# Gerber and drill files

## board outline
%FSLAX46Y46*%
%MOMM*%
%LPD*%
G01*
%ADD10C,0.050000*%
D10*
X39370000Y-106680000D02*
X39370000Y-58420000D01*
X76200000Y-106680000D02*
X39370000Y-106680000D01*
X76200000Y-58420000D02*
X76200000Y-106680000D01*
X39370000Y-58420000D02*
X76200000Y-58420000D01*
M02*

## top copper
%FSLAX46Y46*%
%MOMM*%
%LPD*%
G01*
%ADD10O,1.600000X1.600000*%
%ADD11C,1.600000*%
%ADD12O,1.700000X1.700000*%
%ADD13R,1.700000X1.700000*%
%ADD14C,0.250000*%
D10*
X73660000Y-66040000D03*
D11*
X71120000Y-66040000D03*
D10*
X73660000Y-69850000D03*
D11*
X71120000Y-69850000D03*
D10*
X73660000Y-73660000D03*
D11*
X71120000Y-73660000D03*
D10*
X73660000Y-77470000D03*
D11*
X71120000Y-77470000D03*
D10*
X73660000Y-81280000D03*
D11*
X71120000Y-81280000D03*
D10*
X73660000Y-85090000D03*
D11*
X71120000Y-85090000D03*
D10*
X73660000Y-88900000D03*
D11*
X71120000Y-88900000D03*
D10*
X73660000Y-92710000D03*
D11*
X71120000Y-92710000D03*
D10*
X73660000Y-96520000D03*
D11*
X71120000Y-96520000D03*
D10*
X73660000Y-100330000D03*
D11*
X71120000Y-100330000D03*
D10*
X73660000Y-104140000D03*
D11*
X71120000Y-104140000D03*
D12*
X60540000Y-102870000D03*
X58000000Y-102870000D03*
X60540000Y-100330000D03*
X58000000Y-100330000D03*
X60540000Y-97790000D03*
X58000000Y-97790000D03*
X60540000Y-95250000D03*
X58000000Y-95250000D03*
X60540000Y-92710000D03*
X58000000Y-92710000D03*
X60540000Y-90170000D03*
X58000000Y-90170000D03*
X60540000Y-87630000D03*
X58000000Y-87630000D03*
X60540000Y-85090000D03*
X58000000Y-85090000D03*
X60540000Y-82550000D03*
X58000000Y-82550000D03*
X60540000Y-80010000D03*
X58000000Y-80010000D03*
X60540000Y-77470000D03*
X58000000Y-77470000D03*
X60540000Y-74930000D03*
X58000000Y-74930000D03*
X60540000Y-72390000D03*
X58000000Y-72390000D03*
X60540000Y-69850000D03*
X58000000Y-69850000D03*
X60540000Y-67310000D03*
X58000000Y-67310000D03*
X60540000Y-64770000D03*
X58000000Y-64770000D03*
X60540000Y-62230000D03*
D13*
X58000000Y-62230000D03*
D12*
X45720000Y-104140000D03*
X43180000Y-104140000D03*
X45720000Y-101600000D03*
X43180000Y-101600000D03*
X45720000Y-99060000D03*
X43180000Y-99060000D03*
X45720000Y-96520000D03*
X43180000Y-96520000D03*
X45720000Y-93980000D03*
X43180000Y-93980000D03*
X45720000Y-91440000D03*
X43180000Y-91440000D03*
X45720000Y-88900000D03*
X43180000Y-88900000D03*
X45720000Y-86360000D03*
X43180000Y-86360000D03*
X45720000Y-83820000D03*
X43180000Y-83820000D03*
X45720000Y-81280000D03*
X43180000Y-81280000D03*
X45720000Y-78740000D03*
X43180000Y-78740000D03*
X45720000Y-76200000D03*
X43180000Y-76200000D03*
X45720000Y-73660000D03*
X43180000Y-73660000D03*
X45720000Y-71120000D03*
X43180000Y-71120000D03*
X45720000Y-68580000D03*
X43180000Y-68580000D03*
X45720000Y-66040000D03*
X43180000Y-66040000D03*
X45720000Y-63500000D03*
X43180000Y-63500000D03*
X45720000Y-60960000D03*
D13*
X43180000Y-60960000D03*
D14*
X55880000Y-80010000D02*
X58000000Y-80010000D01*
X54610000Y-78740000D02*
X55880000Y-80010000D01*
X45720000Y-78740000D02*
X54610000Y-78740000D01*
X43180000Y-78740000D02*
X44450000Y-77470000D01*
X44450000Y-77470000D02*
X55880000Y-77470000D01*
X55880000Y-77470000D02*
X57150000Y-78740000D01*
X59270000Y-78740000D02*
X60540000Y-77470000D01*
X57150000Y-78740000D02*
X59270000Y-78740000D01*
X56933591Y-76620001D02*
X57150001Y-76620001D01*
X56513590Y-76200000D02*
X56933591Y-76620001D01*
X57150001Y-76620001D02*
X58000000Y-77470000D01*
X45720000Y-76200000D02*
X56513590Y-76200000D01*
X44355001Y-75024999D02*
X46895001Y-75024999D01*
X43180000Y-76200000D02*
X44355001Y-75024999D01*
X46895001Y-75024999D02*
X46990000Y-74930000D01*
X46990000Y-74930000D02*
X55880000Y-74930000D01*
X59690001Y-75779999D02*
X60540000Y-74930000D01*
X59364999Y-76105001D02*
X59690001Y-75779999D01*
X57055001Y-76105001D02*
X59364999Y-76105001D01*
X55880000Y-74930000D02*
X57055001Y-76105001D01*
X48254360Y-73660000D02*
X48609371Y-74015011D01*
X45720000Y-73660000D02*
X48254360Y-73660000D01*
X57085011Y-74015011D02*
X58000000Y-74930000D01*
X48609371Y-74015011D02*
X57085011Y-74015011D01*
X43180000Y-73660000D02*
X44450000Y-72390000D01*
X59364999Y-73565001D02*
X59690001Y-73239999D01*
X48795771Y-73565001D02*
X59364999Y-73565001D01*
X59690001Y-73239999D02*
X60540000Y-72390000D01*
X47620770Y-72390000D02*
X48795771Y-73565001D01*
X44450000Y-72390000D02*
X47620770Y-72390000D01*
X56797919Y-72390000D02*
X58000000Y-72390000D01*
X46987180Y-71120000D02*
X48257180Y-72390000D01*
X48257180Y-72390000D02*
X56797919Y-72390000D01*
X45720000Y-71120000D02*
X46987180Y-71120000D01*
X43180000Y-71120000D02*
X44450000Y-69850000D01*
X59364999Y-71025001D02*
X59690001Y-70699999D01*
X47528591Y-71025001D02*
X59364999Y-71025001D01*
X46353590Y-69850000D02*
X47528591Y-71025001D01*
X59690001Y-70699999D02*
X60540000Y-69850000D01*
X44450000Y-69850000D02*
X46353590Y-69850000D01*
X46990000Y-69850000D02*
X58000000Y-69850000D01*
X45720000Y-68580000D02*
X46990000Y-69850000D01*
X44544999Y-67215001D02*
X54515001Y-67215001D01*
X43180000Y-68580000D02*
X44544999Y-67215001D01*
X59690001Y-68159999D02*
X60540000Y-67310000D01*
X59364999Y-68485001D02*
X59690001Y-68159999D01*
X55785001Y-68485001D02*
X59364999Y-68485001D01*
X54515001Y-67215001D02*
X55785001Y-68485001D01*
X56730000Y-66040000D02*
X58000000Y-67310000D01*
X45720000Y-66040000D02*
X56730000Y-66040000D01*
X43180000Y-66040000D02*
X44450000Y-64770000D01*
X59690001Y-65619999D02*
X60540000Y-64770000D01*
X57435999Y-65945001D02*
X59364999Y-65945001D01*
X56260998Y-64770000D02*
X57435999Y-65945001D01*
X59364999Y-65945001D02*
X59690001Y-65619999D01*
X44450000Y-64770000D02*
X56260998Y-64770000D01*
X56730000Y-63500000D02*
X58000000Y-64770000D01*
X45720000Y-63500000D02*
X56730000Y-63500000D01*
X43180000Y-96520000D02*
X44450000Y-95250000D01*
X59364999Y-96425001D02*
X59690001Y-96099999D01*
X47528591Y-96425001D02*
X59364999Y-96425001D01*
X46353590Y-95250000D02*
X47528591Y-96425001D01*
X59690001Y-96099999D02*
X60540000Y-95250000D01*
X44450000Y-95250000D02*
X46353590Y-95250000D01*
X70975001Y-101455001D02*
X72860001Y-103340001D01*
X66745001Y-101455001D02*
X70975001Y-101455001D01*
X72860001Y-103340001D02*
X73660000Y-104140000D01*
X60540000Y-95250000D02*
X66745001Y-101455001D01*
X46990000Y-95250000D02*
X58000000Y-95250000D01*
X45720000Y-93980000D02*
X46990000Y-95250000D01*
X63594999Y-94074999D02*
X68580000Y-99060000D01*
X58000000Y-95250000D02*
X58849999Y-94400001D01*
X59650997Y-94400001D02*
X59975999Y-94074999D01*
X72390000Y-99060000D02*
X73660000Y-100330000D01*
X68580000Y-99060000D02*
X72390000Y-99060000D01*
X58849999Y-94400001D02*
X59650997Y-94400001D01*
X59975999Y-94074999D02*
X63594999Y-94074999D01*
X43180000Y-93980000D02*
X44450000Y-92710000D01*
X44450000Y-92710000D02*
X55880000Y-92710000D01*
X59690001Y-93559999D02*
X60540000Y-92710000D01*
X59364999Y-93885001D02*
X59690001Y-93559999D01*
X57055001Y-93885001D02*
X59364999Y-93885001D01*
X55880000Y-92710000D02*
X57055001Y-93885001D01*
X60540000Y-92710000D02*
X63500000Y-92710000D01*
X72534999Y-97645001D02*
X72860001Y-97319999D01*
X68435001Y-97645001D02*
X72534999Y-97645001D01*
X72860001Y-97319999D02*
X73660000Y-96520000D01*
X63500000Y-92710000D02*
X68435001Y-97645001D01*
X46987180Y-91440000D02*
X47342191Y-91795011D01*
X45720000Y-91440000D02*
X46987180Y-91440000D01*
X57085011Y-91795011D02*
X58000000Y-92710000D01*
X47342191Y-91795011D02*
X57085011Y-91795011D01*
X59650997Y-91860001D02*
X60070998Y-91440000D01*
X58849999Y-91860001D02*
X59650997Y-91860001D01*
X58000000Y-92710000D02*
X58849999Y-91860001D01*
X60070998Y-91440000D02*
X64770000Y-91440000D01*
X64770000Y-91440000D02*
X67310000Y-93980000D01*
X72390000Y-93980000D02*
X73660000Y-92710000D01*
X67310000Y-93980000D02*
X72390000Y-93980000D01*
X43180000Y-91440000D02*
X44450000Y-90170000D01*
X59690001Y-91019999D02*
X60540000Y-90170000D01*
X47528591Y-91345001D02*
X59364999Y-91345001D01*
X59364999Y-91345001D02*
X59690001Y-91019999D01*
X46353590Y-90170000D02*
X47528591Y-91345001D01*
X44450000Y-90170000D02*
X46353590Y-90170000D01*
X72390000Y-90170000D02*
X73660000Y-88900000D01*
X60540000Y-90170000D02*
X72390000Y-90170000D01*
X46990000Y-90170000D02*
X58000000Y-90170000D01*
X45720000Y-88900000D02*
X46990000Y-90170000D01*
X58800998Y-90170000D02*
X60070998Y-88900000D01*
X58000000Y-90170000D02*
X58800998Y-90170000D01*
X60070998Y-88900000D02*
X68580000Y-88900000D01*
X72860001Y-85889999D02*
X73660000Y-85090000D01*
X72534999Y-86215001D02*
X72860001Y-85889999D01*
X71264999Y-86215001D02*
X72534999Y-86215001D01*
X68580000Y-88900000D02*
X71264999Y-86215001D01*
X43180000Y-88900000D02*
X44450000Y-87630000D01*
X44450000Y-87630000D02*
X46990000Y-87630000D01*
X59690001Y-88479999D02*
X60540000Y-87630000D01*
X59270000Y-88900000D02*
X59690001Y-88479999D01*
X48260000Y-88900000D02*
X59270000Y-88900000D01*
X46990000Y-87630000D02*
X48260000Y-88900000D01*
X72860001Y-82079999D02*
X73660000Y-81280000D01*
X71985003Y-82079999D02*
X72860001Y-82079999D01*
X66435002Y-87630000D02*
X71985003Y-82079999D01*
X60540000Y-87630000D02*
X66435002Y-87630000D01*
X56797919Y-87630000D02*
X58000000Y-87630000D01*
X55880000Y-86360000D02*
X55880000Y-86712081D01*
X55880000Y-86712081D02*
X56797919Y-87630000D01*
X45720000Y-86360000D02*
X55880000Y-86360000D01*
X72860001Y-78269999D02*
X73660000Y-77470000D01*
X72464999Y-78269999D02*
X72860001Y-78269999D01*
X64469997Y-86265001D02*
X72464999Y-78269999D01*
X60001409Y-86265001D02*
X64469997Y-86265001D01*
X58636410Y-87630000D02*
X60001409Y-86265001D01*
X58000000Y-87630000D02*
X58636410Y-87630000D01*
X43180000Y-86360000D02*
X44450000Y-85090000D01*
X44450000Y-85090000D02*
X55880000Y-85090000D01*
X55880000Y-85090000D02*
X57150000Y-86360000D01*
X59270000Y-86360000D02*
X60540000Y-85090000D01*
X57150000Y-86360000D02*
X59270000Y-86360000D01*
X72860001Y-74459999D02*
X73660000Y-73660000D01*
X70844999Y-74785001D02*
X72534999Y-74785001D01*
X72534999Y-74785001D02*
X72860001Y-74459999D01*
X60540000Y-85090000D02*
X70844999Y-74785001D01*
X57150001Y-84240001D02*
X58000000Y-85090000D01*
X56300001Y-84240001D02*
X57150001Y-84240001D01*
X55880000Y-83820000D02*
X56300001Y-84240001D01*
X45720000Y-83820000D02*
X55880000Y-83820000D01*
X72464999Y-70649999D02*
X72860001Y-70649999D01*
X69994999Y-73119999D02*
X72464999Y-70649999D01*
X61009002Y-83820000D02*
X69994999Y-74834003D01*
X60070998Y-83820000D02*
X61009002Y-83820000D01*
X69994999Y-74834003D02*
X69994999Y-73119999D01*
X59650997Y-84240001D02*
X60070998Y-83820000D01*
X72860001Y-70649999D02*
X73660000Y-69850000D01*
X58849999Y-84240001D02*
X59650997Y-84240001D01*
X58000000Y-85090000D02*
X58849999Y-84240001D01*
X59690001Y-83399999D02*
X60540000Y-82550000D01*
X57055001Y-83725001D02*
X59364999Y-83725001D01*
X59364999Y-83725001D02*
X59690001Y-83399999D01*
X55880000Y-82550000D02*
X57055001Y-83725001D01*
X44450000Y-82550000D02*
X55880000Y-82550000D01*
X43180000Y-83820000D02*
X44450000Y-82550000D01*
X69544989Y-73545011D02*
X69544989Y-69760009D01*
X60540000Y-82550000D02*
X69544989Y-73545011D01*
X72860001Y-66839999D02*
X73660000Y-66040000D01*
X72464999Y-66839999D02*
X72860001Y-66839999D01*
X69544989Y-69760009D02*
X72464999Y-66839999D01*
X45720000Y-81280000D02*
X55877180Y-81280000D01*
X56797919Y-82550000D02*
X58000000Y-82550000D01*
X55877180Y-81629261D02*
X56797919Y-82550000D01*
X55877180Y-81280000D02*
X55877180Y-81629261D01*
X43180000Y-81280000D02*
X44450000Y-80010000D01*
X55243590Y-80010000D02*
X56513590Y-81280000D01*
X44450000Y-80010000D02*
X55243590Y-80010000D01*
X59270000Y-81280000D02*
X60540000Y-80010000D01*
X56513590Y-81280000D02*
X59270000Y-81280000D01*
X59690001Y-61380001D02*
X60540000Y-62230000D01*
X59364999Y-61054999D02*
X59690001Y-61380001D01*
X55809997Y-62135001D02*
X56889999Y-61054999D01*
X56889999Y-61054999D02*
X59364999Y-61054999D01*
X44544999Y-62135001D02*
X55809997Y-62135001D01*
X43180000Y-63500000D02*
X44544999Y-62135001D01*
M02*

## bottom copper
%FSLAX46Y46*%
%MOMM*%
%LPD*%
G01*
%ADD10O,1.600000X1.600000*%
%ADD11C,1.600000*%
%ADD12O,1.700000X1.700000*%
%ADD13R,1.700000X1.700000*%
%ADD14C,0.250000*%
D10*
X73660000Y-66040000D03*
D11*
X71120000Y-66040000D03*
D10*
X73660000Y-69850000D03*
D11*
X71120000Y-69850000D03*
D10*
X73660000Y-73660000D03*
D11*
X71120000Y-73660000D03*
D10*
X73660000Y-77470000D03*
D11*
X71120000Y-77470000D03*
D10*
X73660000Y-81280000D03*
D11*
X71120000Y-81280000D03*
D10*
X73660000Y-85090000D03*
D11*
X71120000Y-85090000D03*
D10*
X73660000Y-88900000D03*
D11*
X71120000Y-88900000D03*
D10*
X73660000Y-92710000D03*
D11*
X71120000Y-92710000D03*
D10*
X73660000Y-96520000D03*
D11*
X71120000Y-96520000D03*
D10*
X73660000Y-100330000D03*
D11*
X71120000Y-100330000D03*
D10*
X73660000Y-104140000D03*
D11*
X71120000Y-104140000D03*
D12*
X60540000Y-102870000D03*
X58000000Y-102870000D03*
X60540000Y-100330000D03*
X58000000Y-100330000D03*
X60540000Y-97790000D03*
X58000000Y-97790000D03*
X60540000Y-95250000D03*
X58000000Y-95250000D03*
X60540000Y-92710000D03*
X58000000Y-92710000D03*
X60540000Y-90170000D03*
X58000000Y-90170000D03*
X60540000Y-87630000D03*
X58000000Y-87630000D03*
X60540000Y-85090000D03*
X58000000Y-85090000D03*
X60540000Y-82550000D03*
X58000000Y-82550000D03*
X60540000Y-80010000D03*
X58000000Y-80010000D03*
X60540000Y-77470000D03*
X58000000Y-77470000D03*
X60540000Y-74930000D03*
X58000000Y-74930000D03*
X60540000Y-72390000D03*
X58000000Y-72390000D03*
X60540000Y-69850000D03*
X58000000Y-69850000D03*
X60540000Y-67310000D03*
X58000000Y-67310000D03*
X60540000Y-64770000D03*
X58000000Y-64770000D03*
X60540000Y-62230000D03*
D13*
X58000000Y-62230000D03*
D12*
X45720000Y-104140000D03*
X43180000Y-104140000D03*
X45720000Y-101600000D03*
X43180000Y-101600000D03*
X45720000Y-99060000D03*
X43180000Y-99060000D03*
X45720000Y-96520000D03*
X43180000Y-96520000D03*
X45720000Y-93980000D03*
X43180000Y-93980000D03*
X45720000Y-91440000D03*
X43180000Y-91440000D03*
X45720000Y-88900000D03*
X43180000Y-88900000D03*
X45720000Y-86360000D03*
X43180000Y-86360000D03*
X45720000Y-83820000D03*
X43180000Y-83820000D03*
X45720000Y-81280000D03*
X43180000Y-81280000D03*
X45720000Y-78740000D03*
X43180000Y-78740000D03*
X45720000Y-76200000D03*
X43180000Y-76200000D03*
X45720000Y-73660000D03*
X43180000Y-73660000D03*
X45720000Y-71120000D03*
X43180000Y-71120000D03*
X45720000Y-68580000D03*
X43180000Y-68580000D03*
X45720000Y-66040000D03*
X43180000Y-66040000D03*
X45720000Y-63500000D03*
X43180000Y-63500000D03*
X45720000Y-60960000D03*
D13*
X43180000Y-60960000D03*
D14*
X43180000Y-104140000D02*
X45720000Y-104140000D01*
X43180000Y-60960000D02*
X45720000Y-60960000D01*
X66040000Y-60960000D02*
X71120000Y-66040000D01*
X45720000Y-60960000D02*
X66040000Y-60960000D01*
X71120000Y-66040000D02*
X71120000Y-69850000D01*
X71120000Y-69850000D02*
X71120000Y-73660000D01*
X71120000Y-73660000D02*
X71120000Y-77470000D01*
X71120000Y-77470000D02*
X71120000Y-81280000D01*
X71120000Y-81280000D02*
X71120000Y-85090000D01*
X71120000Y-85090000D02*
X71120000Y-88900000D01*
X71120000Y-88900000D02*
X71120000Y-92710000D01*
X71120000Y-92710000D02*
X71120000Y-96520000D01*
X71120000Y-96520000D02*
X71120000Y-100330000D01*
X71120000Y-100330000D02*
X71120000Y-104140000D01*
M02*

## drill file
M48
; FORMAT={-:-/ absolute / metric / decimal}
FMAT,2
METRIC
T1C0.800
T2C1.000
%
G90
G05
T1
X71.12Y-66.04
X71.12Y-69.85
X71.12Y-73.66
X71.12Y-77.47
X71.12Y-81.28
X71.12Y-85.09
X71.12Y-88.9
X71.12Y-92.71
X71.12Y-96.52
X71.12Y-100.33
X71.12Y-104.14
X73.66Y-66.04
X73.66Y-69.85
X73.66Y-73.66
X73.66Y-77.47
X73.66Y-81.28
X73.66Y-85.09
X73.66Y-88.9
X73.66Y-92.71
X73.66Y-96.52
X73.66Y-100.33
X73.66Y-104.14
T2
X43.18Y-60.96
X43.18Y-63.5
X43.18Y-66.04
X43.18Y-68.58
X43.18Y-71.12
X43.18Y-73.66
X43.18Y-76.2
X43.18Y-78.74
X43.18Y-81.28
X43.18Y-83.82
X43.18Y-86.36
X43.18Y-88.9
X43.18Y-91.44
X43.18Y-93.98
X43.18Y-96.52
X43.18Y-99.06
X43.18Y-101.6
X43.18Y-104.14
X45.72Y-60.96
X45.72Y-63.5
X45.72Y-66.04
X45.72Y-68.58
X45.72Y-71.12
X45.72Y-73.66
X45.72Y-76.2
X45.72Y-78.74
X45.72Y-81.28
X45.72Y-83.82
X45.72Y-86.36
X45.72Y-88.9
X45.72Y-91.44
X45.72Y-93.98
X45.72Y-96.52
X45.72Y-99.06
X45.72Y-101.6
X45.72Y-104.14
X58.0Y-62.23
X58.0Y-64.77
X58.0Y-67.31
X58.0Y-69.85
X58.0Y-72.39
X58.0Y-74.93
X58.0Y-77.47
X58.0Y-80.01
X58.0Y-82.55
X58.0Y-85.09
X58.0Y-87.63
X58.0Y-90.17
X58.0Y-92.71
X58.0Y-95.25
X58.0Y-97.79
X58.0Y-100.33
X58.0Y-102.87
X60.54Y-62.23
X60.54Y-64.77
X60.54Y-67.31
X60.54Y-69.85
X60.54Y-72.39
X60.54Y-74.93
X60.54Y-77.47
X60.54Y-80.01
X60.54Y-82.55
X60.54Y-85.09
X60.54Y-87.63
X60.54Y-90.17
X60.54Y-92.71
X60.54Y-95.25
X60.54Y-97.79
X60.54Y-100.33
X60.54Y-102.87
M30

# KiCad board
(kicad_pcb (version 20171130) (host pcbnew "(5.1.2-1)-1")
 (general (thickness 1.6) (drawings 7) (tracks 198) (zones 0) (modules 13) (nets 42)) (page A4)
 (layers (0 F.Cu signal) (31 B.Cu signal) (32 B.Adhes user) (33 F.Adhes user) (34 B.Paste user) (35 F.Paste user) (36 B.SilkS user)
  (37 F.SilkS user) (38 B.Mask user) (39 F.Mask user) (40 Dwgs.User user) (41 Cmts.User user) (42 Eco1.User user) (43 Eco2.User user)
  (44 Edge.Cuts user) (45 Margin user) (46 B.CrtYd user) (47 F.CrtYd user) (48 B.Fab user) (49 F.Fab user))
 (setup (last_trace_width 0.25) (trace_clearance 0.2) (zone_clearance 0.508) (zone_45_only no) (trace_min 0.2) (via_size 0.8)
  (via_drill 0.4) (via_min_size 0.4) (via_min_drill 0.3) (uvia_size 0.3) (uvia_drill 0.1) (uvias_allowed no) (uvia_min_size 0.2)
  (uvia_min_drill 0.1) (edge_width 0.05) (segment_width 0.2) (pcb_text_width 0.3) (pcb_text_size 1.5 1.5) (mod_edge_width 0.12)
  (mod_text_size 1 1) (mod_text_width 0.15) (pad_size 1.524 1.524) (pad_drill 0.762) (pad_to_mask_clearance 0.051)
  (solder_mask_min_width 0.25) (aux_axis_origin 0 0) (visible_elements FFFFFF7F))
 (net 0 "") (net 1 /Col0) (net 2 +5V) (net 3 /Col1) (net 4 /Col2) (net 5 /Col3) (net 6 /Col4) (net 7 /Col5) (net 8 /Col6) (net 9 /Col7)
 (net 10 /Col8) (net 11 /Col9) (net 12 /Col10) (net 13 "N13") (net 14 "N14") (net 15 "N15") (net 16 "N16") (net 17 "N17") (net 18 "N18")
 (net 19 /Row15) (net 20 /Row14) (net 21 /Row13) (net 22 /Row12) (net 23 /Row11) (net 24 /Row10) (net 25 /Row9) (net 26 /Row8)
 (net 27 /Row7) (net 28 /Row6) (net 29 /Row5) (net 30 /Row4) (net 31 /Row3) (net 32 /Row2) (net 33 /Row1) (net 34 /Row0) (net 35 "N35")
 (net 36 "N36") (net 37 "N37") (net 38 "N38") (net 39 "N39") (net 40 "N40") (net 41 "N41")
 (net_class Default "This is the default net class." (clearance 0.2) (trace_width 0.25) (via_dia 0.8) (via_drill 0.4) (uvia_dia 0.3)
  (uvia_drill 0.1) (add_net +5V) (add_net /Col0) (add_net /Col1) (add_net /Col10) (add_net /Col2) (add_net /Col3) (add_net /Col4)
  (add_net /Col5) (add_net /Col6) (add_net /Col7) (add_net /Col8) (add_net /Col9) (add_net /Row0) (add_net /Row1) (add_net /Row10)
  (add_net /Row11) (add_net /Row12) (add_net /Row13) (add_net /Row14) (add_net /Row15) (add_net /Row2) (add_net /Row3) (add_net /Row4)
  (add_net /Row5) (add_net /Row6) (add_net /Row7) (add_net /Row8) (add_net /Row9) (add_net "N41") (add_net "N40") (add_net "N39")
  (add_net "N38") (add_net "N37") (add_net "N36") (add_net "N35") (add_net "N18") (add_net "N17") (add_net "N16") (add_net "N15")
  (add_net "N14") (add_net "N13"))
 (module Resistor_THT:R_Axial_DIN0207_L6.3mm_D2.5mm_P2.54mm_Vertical (layer F.Cu) (at 71.12 66.04)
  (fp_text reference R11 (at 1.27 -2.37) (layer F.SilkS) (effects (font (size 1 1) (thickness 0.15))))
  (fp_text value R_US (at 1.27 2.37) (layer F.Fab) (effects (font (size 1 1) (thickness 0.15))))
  (pad 2 thru_hole oval (at 2.54 0) (size 1.6 1.6) (drill 0.8) (layers *.Cu *.Mask) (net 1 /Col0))
  (pad 1 thru_hole circle (at 0 0) (size 1.6 1.6) (drill 0.8) (layers *.Cu *.Mask) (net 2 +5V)))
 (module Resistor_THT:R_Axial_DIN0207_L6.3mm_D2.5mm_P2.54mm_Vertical (layer F.Cu) (at 71.12 69.85)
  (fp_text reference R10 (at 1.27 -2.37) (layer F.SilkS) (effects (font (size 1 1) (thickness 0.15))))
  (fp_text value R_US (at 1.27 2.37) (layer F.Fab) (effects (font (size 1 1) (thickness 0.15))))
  (pad 2 thru_hole oval (at 2.54 0) (size 1.6 1.6) (drill 0.8) (layers *.Cu *.Mask) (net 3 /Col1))
  (pad 1 thru_hole circle (at 0 0) (size 1.6 1.6) (drill 0.8) (layers *.Cu *.Mask) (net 2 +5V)))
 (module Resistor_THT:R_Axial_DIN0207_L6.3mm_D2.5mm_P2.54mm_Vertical (layer F.Cu) (at 71.12 73.66)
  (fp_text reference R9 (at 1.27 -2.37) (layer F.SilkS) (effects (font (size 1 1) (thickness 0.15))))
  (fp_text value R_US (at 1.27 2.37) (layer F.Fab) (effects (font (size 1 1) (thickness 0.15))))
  (pad 2 thru_hole oval (at 2.54 0) (size 1.6 1.6) (drill 0.8) (layers *.Cu *.Mask) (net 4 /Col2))
  (pad 1 thru_hole circle (at 0 0) (size 1.6 1.6) (drill 0.8) (layers *.Cu *.Mask) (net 2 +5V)))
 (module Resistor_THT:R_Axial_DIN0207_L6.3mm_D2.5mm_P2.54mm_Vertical (layer F.Cu) (at 71.12 77.47)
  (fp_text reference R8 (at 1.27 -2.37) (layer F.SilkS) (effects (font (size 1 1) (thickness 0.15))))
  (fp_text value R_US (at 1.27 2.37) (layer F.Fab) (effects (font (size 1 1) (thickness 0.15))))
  (pad 2 thru_hole oval (at 2.54 0) (size 1.6 1.6) (drill 0.8) (layers *.Cu *.Mask) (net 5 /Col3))
  (pad 1 thru_hole circle (at 0 0) (size 1.6 1.6) (drill 0.8) (layers *.Cu *.Mask) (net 2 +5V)))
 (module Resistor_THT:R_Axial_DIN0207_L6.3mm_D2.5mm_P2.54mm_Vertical (layer F.Cu) (at 71.12 81.28)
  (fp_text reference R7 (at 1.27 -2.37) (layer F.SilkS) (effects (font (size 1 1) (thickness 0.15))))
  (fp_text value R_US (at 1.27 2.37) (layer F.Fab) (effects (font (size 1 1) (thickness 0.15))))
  (pad 2 thru_hole oval (at 2.54 0) (size 1.6 1.6) (drill 0.8) (layers *.Cu *.Mask) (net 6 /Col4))
  (pad 1 thru_hole circle (at 0 0) (size 1.6 1.6) (drill 0.8) (layers *.Cu *.Mask) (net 2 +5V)))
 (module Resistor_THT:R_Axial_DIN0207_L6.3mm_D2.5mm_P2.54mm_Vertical (layer F.Cu) (at 71.12 85.09)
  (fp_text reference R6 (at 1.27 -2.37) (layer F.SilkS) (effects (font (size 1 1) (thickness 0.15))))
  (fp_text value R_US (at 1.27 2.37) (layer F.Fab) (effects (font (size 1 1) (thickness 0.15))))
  (pad 2 thru_hole oval (at 2.54 0) (size 1.6 1.6) (drill 0.8) (layers *.Cu *.Mask) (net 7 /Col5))
  (pad 1 thru_hole circle (at 0 0) (size 1.6 1.6) (drill 0.8) (layers *.Cu *.Mask) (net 2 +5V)))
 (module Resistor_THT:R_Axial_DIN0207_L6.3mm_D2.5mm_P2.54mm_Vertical (layer F.Cu) (at 71.12 88.9)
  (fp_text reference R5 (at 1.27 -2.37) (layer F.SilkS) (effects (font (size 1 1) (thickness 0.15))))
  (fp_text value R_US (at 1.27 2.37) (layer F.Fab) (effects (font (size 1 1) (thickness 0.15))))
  (pad 2 thru_hole oval (at 2.54 0) (size 1.6 1.6) (drill 0.8) (layers *.Cu *.Mask) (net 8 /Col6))
  (pad 1 thru_hole circle (at 0 0) (size 1.6 1.6) (drill 0.8) (layers *.Cu *.Mask) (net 2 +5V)))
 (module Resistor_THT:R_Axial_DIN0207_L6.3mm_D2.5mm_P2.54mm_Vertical (layer F.Cu) (at 71.12 92.71)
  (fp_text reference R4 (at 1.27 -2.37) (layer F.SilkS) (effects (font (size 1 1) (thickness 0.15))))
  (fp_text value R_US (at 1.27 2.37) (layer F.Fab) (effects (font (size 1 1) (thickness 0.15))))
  (pad 2 thru_hole oval (at 2.54 0) (size 1.6 1.6) (drill 0.8) (layers *.Cu *.Mask) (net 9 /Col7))
  (pad 1 thru_hole circle (at 0 0) (size 1.6 1.6) (drill 0.8) (layers *.Cu *.Mask) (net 2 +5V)))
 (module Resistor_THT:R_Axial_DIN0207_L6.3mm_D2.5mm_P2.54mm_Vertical (layer F.Cu) (at 71.12 96.52)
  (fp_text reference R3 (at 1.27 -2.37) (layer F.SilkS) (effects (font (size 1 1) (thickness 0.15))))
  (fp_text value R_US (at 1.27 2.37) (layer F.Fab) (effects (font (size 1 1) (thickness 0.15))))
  (pad 2 thru_hole oval (at 2.54 0) (size 1.6 1.6) (drill 0.8) (layers *.Cu *.Mask) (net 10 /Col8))
  (pad 1 thru_hole circle (at 0 0) (size 1.6 1.6) (drill 0.8) (layers *.Cu *.Mask) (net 2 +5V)))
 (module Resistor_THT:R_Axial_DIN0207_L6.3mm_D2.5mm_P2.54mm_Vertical (layer F.Cu) (at 71.12 100.33)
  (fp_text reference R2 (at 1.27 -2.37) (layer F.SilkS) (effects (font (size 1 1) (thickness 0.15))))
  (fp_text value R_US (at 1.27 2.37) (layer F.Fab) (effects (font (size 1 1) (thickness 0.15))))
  (pad 2 thru_hole oval (at 2.54 0) (size 1.6 1.6) (drill 0.8) (layers *.Cu *.Mask) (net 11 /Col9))
  (pad 1 thru_hole circle (at 0 0) (size 1.6 1.6) (drill 0.8) (layers *.Cu *.Mask) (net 2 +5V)))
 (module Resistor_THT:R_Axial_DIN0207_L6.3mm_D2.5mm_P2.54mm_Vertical (layer F.Cu) (at 71.12 104.14)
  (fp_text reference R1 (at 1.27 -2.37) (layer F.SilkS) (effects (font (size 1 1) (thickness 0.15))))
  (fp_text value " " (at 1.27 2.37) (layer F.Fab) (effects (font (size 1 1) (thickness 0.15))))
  (pad 2 thru_hole oval (at 2.54 0) (size 1.6 1.6) (drill 0.8) (layers *.Cu *.Mask) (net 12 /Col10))
  (pad 1 thru_hole circle (at 0 0) (size 1.6 1.6) (drill 0.8) (layers *.Cu *.Mask) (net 2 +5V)))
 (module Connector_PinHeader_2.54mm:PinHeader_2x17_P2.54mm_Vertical (layer F.Cu) (at 58 62.23)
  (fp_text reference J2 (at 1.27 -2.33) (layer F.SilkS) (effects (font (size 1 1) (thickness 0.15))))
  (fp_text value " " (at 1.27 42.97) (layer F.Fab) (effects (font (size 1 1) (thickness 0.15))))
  (pad 34 thru_hole oval (at 2.54 40.64) (size 1.7 1.7) (drill 1) (layers *.Cu *.Mask) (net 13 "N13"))
  (pad 33 thru_hole oval (at 0 40.64) (size 1.7 1.7) (drill 1) (layers *.Cu *.Mask) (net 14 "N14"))
  (pad 32 thru_hole oval (at 2.54 38.1) (size 1.7 1.7) (drill 1) (layers *.Cu *.Mask) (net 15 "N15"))
  (pad 31 thru_hole oval (at 0 38.1) (size 1.7 1.7) (drill 1) (layers *.Cu *.Mask) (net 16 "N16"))
  (pad 30 thru_hole oval (at 2.54 35.56) (size 1.7 1.7) (drill 1) (layers *.Cu *.Mask) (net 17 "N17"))
  (pad 29 thru_hole oval (at 0 35.56) (size 1.7 1.7) (drill 1) (layers *.Cu *.Mask) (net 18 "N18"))
  (pad 28 thru_hole oval (at 2.54 33.02) (size 1.7 1.7) (drill 1) (layers *.Cu *.Mask) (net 12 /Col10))
  (pad 27 thru_hole oval (at 0 33.02) (size 1.7 1.7) (drill 1) (layers *.Cu *.Mask) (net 11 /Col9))
  (pad 26 thru_hole oval (at 2.54 30.48) (size 1.7 1.7) (drill 1) (layers *.Cu *.Mask) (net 10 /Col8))
  (pad 25 thru_hole oval (at 0 30.48) (size 1.7 1.7) (drill 1) (layers *.Cu *.Mask) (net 9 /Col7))
  (pad 24 thru_hole oval (at 2.54 27.94) (size 1.7 1.7) (drill 1) (layers *.Cu *.Mask) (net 8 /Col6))
  (pad 23 thru_hole oval (at 0 27.94) (size 1.7 1.7) (drill 1) (layers *.Cu *.Mask) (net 7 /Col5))
  (pad 22 thru_hole oval (at 2.54 25.4) (size 1.7 1.7) (drill 1) (layers *.Cu *.Mask) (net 6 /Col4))
  (pad 21 thru_hole oval (at 0 25.4) (size 1.7 1.7) (drill 1) (layers *.Cu *.Mask) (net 5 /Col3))
  (pad 20 thru_hole oval (at 2.54 22.86) (size 1.7 1.7) (drill 1) (layers *.Cu *.Mask) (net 4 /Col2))
  (pad 19 thru_hole oval (at 0 22.86) (size 1.7 1.7) (drill 1) (layers *.Cu *.Mask) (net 3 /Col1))
  (pad 18 thru_hole oval (at 2.54 20.32) (size 1.7 1.7) (drill 1) (layers *.Cu *.Mask) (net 1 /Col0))
  (pad 17 thru_hole oval (at 0 20.32) (size 1.7 1.7) (drill 1) (layers *.Cu *.Mask) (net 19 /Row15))
  (pad 16 thru_hole oval (at 2.54 17.78) (size 1.7 1.7) (drill 1) (layers *.Cu *.Mask) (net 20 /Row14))
  (pad 15 thru_hole oval (at 0 17.78) (size 1.7 1.7) (drill 1) (layers *.Cu *.Mask) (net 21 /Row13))
  (pad 14 thru_hole oval (at 2.54 15.24) (size 1.7 1.7) (drill 1) (layers *.Cu *.Mask) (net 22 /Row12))
  (pad 13 thru_hole oval (at 0 15.24) (size 1.7 1.7) (drill 1) (layers *.Cu *.Mask) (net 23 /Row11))
  (pad 12 thru_hole oval (at 2.54 12.7) (size 1.7 1.7) (drill 1) (layers *.Cu *.Mask) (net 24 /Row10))
  (pad 11 thru_hole oval (at 0 12.7) (size 1.7 1.7) (drill 1) (layers *.Cu *.Mask) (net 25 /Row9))
  (pad 10 thru_hole oval (at 2.54 10.16) (size 1.7 1.7) (drill 1) (layers *.Cu *.Mask) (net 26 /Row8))
  (pad 9 thru_hole oval (at 0 10.16) (size 1.7 1.7) (drill 1) (layers *.Cu *.Mask) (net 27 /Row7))
  (pad 8 thru_hole oval (at 2.54 7.62) (size 1.7 1.7) (drill 1) (layers *.Cu *.Mask) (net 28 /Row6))
  (pad 7 thru_hole oval (at 0 7.62) (size 1.7 1.7) (drill 1) (layers *.Cu *.Mask) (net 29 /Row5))
  (pad 6 thru_hole oval (at 2.54 5.08) (size 1.7 1.7) (drill 1) (layers *.Cu *.Mask) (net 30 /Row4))
  (pad 5 thru_hole oval (at 0 5.08) (size 1.7 1.7) (drill 1) (layers *.Cu *.Mask) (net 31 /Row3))
  (pad 4 thru_hole oval (at 2.54 2.54) (size 1.7 1.7) (drill 1) (layers *.Cu *.Mask) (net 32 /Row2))
  (pad 3 thru_hole oval (at 0 2.54) (size 1.7 1.7) (drill 1) (layers *.Cu *.Mask) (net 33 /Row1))
  (pad 2 thru_hole oval (at 2.54 0) (size 1.7 1.7) (drill 1) (layers *.Cu *.Mask) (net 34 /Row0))
  (pad 1 thru_hole rect (at 0 0) (size 1.7 1.7) (drill 1) (layers *.Cu *.Mask) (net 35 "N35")))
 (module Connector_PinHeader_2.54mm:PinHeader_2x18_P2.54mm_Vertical (layer F.Cu) (at 43.18 60.96)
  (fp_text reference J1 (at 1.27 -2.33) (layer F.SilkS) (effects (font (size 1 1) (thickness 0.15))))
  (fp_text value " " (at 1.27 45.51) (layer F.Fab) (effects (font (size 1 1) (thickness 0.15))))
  (pad 36 thru_hole oval (at 2.54 43.18) (size 1.7 1.7) (drill 1) (layers *.Cu *.Mask) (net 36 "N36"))
  (pad 35 thru_hole oval (at 0 43.18) (size 1.7 1.7) (drill 1) (layers *.Cu *.Mask) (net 36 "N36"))
  (pad 34 thru_hole oval (at 2.54 40.64) (size 1.7 1.7) (drill 1) (layers *.Cu *.Mask) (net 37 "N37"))
  (pad 33 thru_hole oval (at 0 40.64) (size 1.7 1.7) (drill 1) (layers *.Cu *.Mask) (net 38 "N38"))
  (pad 32 thru_hole oval (at 2.54 38.1) (size 1.7 1.7) (drill 1) (layers *.Cu *.Mask) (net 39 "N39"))
  (pad 31 thru_hole oval (at 0 38.1) (size 1.7 1.7) (drill 1) (layers *.Cu *.Mask) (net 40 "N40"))
  (pad 30 thru_hole oval (at 2.54 35.56) (size 1.7 1.7) (drill 1) (layers *.Cu *.Mask) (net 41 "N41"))
  (pad 29 thru_hole oval (at 0 35.56) (size 1.7 1.7) (drill 1) (layers *.Cu *.Mask) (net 12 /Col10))
  (pad 28 thru_hole oval (at 2.54 33.02) (size 1.7 1.7) (drill 1) (layers *.Cu *.Mask) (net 11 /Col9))
  (pad 27 thru_hole oval (at 0 33.02) (size 1.7 1.7) (drill 1) (layers *.Cu *.Mask) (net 10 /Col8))
  (pad 26 thru_hole oval (at 2.54 30.48) (size 1.7 1.7) (drill 1) (layers *.Cu *.Mask) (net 9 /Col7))
  (pad 25 thru_hole oval (at 0 30.48) (size 1.7 1.7) (drill 1) (layers *.Cu *.Mask) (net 8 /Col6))
  (pad 24 thru_hole oval (at 2.54 27.94) (size 1.7 1.7) (drill 1) (layers *.Cu *.Mask) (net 7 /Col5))
  (pad 23 thru_hole oval (at 0 27.94) (size 1.7 1.7) (drill 1) (layers *.Cu *.Mask) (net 6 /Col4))
  (pad 22 thru_hole oval (at 2.54 25.4) (size 1.7 1.7) (drill 1) (layers *.Cu *.Mask) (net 5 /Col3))
  (pad 21 thru_hole oval (at 0 25.4) (size 1.7 1.7) (drill 1) (layers *.Cu *.Mask) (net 4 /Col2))
  (pad 20 thru_hole oval (at 2.54 22.86) (size 1.7 1.7) (drill 1) (layers *.Cu *.Mask) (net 3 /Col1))
  (pad 19 thru_hole oval (at 0 22.86) (size 1.7 1.7) (drill 1) (layers *.Cu *.Mask) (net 1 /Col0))
  (pad 18 thru_hole oval (at 2.54 20.32) (size 1.7 1.7) (drill 1) (layers *.Cu *.Mask) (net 19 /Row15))
  (pad 17 thru_hole oval (at 0 20.32) (size 1.7 1.7) (drill 1) (layers *.Cu *.Mask) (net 20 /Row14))
  (pad 16 thru_hole oval (at 2.54 17.78) (size 1.7 1.7) (drill 1) (layers *.Cu *.Mask) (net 21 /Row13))
  (pad 15 thru_hole oval (at 0 17.78) (size 1.7 1.7) (drill 1) (layers *.Cu *.Mask) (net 22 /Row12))
  (pad 14 thru_hole oval (at 2.54 15.24) (size 1.7 1.7) (drill 1) (layers *.Cu *.Mask) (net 23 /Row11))
  (pad 13 thru_hole oval (at 0 15.24) (size 1.7 1.7) (drill 1) (layers *.Cu *.Mask) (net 24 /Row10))
  (pad 12 thru_hole oval (at 2.54 12.7) (size 1.7 1.7) (drill 1) (layers *.Cu *.Mask) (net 25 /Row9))
  (pad 11 thru_hole oval (at 0 12.7) (size 1.7 1.7) (drill 1) (layers *.Cu *.Mask) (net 26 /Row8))
  (pad 10 thru_hole oval (at 2.54 10.16) (size 1.7 1.7) (drill 1) (layers *.Cu *.Mask) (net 27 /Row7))
  (pad 9 thru_hole oval (at 0 10.16) (size 1.7 1.7) (drill 1) (layers *.Cu *.Mask) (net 28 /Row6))
  (pad 8 thru_hole oval (at 2.54 7.62) (size 1.7 1.7) (drill 1) (layers *.Cu *.Mask) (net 29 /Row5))
  (pad 7 thru_hole oval (at 0 7.62) (size 1.7 1.7) (drill 1) (layers *.Cu *.Mask) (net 30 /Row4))
  (pad 6 thru_hole oval (at 2.54 5.08) (size 1.7 1.7) (drill 1) (layers *.Cu *.Mask) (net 31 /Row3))
  (pad 5 thru_hole oval (at 0 5.08) (size 1.7 1.7) (drill 1) (layers *.Cu *.Mask) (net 32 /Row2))
  (pad 4 thru_hole oval (at 2.54 2.54) (size 1.7 1.7) (drill 1) (layers *.Cu *.Mask) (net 33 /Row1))
  (pad 3 thru_hole oval (at 0 2.54) (size 1.7 1.7) (drill 1) (layers *.Cu *.Mask) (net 34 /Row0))
  (pad 2 thru_hole oval (at 2.54 0) (size 1.7 1.7) (drill 1) (layers *.Cu *.Mask) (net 2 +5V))
  (pad 1 thru_hole rect (at 0 0) (size 1.7 1.7) (drill 1) (layers *.Cu *.Mask) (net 2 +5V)))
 (gr_line (start 39.37 106.68) (end 39.37 58.42) (layer Edge.Cuts) (width 0.05))
 (gr_line (start 76.2 106.68) (end 39.37 106.68) (layer Edge.Cuts) (width 0.05))
 (gr_line (start 76.2 58.42) (end 76.2 106.68) (layer Edge.Cuts) (width 0.05))
 (gr_line (start 39.37 58.42) (end 76.2 58.42) (layer Edge.Cuts) (width 0.05))
 (segment (start 43.18 104.14) (end 45.72 104.14) (width 0.25) (layer B.Cu) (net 36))
 (segment (start 55.88 80.01) (end 58 80.01) (width 0.25) (layer F.Cu) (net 21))
 (segment (start 54.61 78.74) (end 55.88 80.01) (width 0.25) (layer F.Cu) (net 21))
 (segment (start 45.72 78.74) (end 54.61 78.74) (width 0.25) (layer F.Cu) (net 21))
 (segment (start 43.18 78.74) (end 44.45 77.47) (width 0.25) (layer F.Cu) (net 22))
 (segment (start 44.45 77.47) (end 55.88 77.47) (width 0.25) (layer F.Cu) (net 22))
 (segment (start 55.88 77.47) (end 57.15 78.74) (width 0.25) (layer F.Cu) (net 22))
 (segment (start 59.27 78.74) (end 60.54 77.47) (width 0.25) (layer F.Cu) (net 22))
 (segment (start 57.15 78.74) (end 59.27 78.74) (width 0.25) (layer F.Cu) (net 22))
 (segment (start 56.933591 76.620001) (end 57.150001 76.620001) (width 0.25) (layer F.Cu) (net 23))
 (segment (start 56.51359 76.2) (end 56.933591 76.620001) (width 0.25) (layer F.Cu) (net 23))
 (segment (start 57.150001 76.620001) (end 58 77.47) (width 0.25) (layer F.Cu) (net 23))
 (segment (start 45.72 76.2) (end 56.51359 76.2) (width 0.25) (layer F.Cu) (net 23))
 (segment (start 44.355001 75.024999) (end 46.895001 75.024999) (width 0.25) (layer F.Cu) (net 24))
 (segment (start 43.18 76.2) (end 44.355001 75.024999) (width 0.25) (layer F.Cu) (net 24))
 (segment (start 46.895001 75.024999) (end 46.99 74.93) (width 0.25) (layer F.Cu) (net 24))
 (segment (start 46.99 74.93) (end 55.88 74.93) (width 0.25) (layer F.Cu) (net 24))
 (segment (start 59.690001 75.779999) (end 60.54 74.93) (width 0.25) (layer F.Cu) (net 24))
 (segment (start 59.364999 76.105001) (end 59.690001 75.779999) (width 0.25) (layer F.Cu) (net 24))
 (segment (start 57.055001 76.105001) (end 59.364999 76.105001) (width 0.25) (layer F.Cu) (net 24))
 (segment (start 55.88 74.93) (end 57.055001 76.105001) (width 0.25) (layer F.Cu) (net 24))
 (segment (start 48.25436 73.66) (end 48.609371 74.015011) (width 0.25) (layer F.Cu) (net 25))
 (segment (start 45.72 73.66) (end 48.25436 73.66) (width 0.25) (layer F.Cu) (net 25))
 (segment (start 57.085011 74.015011) (end 58 74.93) (width 0.25) (layer F.Cu) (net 25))
 (segment (start 48.609371 74.015011) (end 57.085011 74.015011) (width 0.25) (layer F.Cu) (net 25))
 (segment (start 43.18 73.66) (end 44.45 72.39) (width 0.25) (layer F.Cu) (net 26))
 (segment (start 59.364999 73.565001) (end 59.690001 73.239999) (width 0.25) (layer F.Cu) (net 26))
 (segment (start 48.795771 73.565001) (end 59.364999 73.565001) (width 0.25) (layer F.Cu) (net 26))
 (segment (start 59.690001 73.239999) (end 60.54 72.39) (width 0.25) (layer F.Cu) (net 26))
 (segment (start 47.62077 72.39) (end 48.795771 73.565001) (width 0.25) (layer F.Cu) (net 26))
 (segment (start 44.45 72.39) (end 47.62077 72.39) (width 0.25) (layer F.Cu) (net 26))
 (segment (start 56.797919 72.39) (end 58 72.39) (width 0.25) (layer F.Cu) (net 27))
 (segment (start 46.98718 71.12) (end 48.25718 72.39) (width 0.25) (layer F.Cu) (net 27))
 (segment (start 48.25718 72.39) (end 56.797919 72.39) (width 0.25) (layer F.Cu) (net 27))
 (segment (start 45.72 71.12) (end 46.98718 71.12) (width 0.25) (layer F.Cu) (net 27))
 (segment (start 43.18 71.12) (end 44.45 69.85) (width 0.25) (layer F.Cu) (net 28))
 (segment (start 59.364999 71.025001) (end 59.690001 70.699999) (width 0.25) (layer F.Cu) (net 28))
 (segment (start 47.528591 71.025001) (end 59.364999 71.025001) (width 0.25) (layer F.Cu) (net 28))
 (segment (start 46.35359 69.85) (end 47.528591 71.025001) (width 0.25) (layer F.Cu) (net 28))
 (segment (start 59.690001 70.699999) (end 60.54 69.85) (width 0.25) (layer F.Cu) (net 28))
 (segment (start 44.45 69.85) (end 46.35359 69.85) (width 0.25) (layer F.Cu) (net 28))
 (segment (start 46.99 69.85) (end 58 69.85) (width 0.25) (layer F.Cu) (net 29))
 (segment (start 45.72 68.58) (end 46.99 69.85) (width 0.25) (layer F.Cu) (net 29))
 (segment (start 44.544999 67.215001) (end 54.515001 67.215001) (width 0.25) (layer F.Cu) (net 30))
 (segment (start 43.18 68.58) (end 44.544999 67.215001) (width 0.25) (layer F.Cu) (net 30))
 (segment (start 59.690001 68.159999) (end 60.54 67.31) (width 0.25) (layer F.Cu) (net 30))
 (segment (start 59.364999 68.485001) (end 59.690001 68.159999) (width 0.25) (layer F.Cu) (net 30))
 (segment (start 55.785001 68.485001) (end 59.364999 68.485001) (width 0.25) (layer F.Cu) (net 30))
 (segment (start 54.515001 67.215001) (end 55.785001 68.485001) (width 0.25) (layer F.Cu) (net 30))
 (segment (start 56.73 66.04) (end 58 67.31) (width 0.25) (layer F.Cu) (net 31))
 (segment (start 45.72 66.04) (end 56.73 66.04) (width 0.25) (layer F.Cu) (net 31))
 (segment (start 43.18 66.04) (end 44.45 64.77) (width 0.25) (layer F.Cu) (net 32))
 (segment (start 59.690001 65.619999) (end 60.54 64.77) (width 0.25) (layer F.Cu) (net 32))
 (segment (start 57.435999 65.945001) (end 59.364999 65.945001) (width 0.25) (layer F.Cu) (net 32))
 (segment (start 56.260998 64.77) (end 57.435999 65.945001) (width 0.25) (layer F.Cu) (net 32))
 (segment (start 59.364999 65.945001) (end 59.690001 65.619999) (width 0.25) (layer F.Cu) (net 32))
 (segment (start 44.45 64.77) (end 56.260998 64.77) (width 0.25) (layer F.Cu) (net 32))
 (segment (start 56.73 63.5) (end 58 64.77) (width 0.25) (layer F.Cu) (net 33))
 (segment (start 45.72 63.5) (end 56.73 63.5) (width 0.25) (layer F.Cu) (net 33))
 (segment (start 43.18 96.52) (end 44.45 95.25) (width 0.25) (layer F.Cu) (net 12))
 (segment (start 59.364999 96.425001) (end 59.690001 96.099999) (width 0.25) (layer F.Cu) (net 12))
 (segment (start 47.528591 96.425001) (end 59.364999 96.425001) (width 0.25) (layer F.Cu) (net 12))
 (segment (start 46.35359 95.25) (end 47.528591 96.425001) (width 0.25) (layer F.Cu) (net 12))
 (segment (start 59.690001 96.099999) (end 60.54 95.25) (width 0.25) (layer F.Cu) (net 12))
 (segment (start 44.45 95.25) (end 46.35359 95.25) (width 0.25) (layer F.Cu) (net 12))
 (segment (start 70.975001 101.455001) (end 72.860001 103.340001) (width 0.25) (layer F.Cu) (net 12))
 (segment (start 66.745001 101.455001) (end 70.975001 101.455001) (width 0.25) (layer F.Cu) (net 12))
 (segment (start 72.860001 103.340001) (end 73.66 104.14) (width 0.25) (layer F.Cu) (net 12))
 (segment (start 60.54 95.25) (end 66.745001 101.455001) (width 0.25) (layer F.Cu) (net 12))
 (segment (start 46.99 95.25) (end 58 95.25) (width 0.25) (layer F.Cu) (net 11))
 (segment (start 45.72 93.98) (end 46.99 95.25) (width 0.25) (layer F.Cu) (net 11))
 (segment (start 63.594999 94.074999) (end 68.58 99.06) (width 0.25) (layer F.Cu) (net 11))
 (segment (start 58 95.25) (end 58.849999 94.400001) (width 0.25) (layer F.Cu) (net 11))
 (segment (start 59.650997 94.400001) (end 59.975999 94.074999) (width 0.25) (layer F.Cu) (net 11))
 (segment (start 72.39 99.06) (end 73.66 100.33) (width 0.25) (layer F.Cu) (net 11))
 (segment (start 68.58 99.06) (end 72.39 99.06) (width 0.25) (layer F.Cu) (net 11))
 (segment (start 58.849999 94.400001) (end 59.650997 94.400001) (width 0.25) (layer F.Cu) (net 11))
 (segment (start 59.975999 94.074999) (end 63.594999 94.074999) (width 0.25) (layer F.Cu) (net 11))
 (segment (start 43.18 93.98) (end 44.45 92.71) (width 0.25) (layer F.Cu) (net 10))
 (segment (start 44.45 92.71) (end 55.88 92.71) (width 0.25) (layer F.Cu) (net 10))
 (segment (start 59.690001 93.559999) (end 60.54 92.71) (width 0.25) (layer F.Cu) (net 10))
 (segment (start 59.364999 93.885001) (end 59.690001 93.559999) (width 0.25) (layer F.Cu) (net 10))
 (segment (start 57.055001 93.885001) (end 59.364999 93.885001) (width 0.25) (layer F.Cu) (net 10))
 (segment (start 55.88 92.71) (end 57.055001 93.885001) (width 0.25) (layer F.Cu) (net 10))
 (segment (start 60.54 92.71) (end 63.5 92.71) (width 0.25) (layer F.Cu) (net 10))
 (segment (start 72.534999 97.645001) (end 72.860001 97.319999) (width 0.25) (layer F.Cu) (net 10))
 (segment (start 68.435001 97.645001) (end 72.534999 97.645001) (width 0.25) (layer F.Cu) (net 10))
 (segment (start 72.860001 97.319999) (end 73.66 96.52) (width 0.25) (layer F.Cu) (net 10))
 (segment (start 63.5 92.71) (end 68.435001 97.645001) (width 0.25) (layer F.Cu) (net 10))
 (segment (start 46.98718 91.44) (end 47.342191 91.795011) (width 0.25) (layer F.Cu) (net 9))
 (segment (start 45.72 91.44) (end 46.98718 91.44) (width 0.25) (layer F.Cu) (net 9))
 (segment (start 57.085011 91.795011) (end 58 92.71) (width 0.25) (layer F.Cu) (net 9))
 (segment (start 47.342191 91.795011) (end 57.085011 91.795011) (width 0.25) (layer F.Cu) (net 9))
 (segment (start 59.650997 91.860001) (end 60.070998 91.44) (width 0.25) (layer F.Cu) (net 9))
 (segment (start 58.849999 91.860001) (end 59.650997 91.860001) (width 0.25) (layer F.Cu) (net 9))
 (segment (start 58 92.71) (end 58.849999 91.860001) (width 0.25) (layer F.Cu) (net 9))
 (segment (start 60.070998 91.44) (end 64.77 91.44) (width 0.25) (layer F.Cu) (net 9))
 (segment (start 64.77 91.44) (end 67.31 93.98) (width 0.25) (layer F.Cu) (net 9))
 (segment (start 72.39 93.98) (end 73.66 92.71) (width 0.25) (layer F.Cu) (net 9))
 (segment (start 67.31 93.98) (end 72.39 93.98) (width 0.25) (layer F.Cu) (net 9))
 (segment (start 43.18 91.44) (end 44.45 90.17) (width 0.25) (layer F.Cu) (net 8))
 (segment (start 59.690001 91.019999) (end 60.54 90.17) (width 0.25) (layer F.Cu) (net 8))
 (segment (start 47.528591 91.345001) (end 59.364999 91.345001) (width 0.25) (layer F.Cu) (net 8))
 (segment (start 59.364999 91.345001) (end 59.690001 91.019999) (width 0.25) (layer F.Cu) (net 8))
 (segment (start 46.35359 90.17) (end 47.528591 91.345001) (width 0.25) (layer F.Cu) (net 8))
 (segment (start 44.45 90.17) (end 46.35359 90.17) (width 0.25) (layer F.Cu) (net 8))
 (segment (start 72.39 90.17) (end 73.66 88.9) (width 0.25) (layer F.Cu) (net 8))
 (segment (start 60.54 90.17) (end 72.39 90.17) (width 0.25) (layer F.Cu) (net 8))
 (segment (start 46.99 90.17) (end 58 90.17) (width 0.25) (layer F.Cu) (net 7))
 (segment (start 45.72 88.9) (end 46.99 90.17) (width 0.25) (layer F.Cu) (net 7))
 (segment (start 58.800998 90.17) (end 60.070998 88.9) (width 0.25) (layer F.Cu) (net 7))
 (segment (start 58 90.17) (end 58.800998 90.17) (width 0.25) (layer F.Cu) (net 7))
 (segment (start 60.070998 88.9) (end 68.58 88.9) (width 0.25) (layer F.Cu) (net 7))
 (segment (start 72.860001 85.889999) (end 73.66 85.09) (width 0.25) (layer F.Cu) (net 7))
 (segment (start 72.534999 86.215001) (end 72.860001 85.889999) (width 0.25) (layer F.Cu) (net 7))
 (segment (start 71.264999 86.215001) (end 72.534999 86.215001) (width 0.25) (layer F.Cu) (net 7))
 (segment (start 68.58 88.9) (end 71.264999 86.215001) (width 0.25) (layer F.Cu) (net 7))
 (segment (start 43.18 88.9) (end 44.45 87.63) (width 0.25) (layer F.Cu) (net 6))
 (segment (start 44.45 87.63) (end 46.99 87.63) (width 0.25) (layer F.Cu) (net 6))
 (segment (start 59.690001 88.479999) (end 60.54 87.63) (width 0.25) (layer F.Cu) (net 6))
 (segment (start 59.27 88.9) (end 59.690001 88.479999) (width 0.25) (layer F.Cu) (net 6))
 (segment (start 48.26 88.9) (end 59.27 88.9) (width 0.25) (layer F.Cu) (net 6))
 (segment (start 46.99 87.63) (end 48.26 88.9) (width 0.25) (layer F.Cu) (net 6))
 (segment (start 72.860001 82.079999) (end 73.66 81.28) (width 0.25) (layer F.Cu) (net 6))
 (segment (start 71.985003 82.079999) (end 72.860001 82.079999) (width 0.25) (layer F.Cu) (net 6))
 (segment (start 66.435002 87.63) (end 71.985003 82.079999) (width 0.25) (layer F.Cu) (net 6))
 (segment (start 60.54 87.63) (end 66.435002 87.63) (width 0.25) (layer F.Cu) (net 6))
 (segment (start 56.797919 87.63) (end 58 87.63) (width 0.25) (layer F.Cu) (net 5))
 (segment (start 55.88 86.36) (end 55.88 86.712081) (width 0.25) (layer F.Cu) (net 5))
 (segment (start 55.88 86.712081) (end 56.797919 87.63) (width 0.25) (layer F.Cu) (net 5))
 (segment (start 45.72 86.36) (end 55.88 86.36) (width 0.25) (layer F.Cu) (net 5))
 (segment (start 72.860001 78.269999) (end 73.66 77.47) (width 0.25) (layer F.Cu) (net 5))
 (segment (start 72.464999 78.269999) (end 72.860001 78.269999) (width 0.25) (layer F.Cu) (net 5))
 (segment (start 64.469997 86.265001) (end 72.464999 78.269999) (width 0.25) (layer F.Cu) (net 5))
 (segment (start 60.001409 86.265001) (end 64.469997 86.265001) (width 0.25) (layer F.Cu) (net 5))
 (segment (start 58.63641 87.63) (end 60.001409 86.265001) (width 0.25) (layer F.Cu) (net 5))
 (segment (start 58 87.63) (end 58.63641 87.63) (width 0.25) (layer F.Cu) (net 5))
 (segment (start 43.18 86.36) (end 44.45 85.09) (width 0.25) (layer F.Cu) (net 4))
 (segment (start 44.45 85.09) (end 55.88 85.09) (width 0.25) (layer F.Cu) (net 4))
 (segment (start 55.88 85.09) (end 57.15 86.36) (width 0.25) (layer F.Cu) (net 4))
 (segment (start 59.27 86.36) (end 60.54 85.09) (width 0.25) (layer F.Cu) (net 4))
 (segment (start 57.15 86.36) (end 59.27 86.36) (width 0.25) (layer F.Cu) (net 4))
 (segment (start 72.860001 74.459999) (end 73.66 73.66) (width 0.25) (layer F.Cu) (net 4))
 (segment (start 70.844999 74.785001) (end 72.534999 74.785001) (width 0.25) (layer F.Cu) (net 4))
 (segment (start 72.534999 74.785001) (end 72.860001 74.459999) (width 0.25) (layer F.Cu) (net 4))
 (segment (start 60.54 85.09) (end 70.844999 74.785001) (width 0.25) (layer F.Cu) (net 4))
 (segment (start 57.150001 84.240001) (end 58 85.09) (width 0.25) (layer F.Cu) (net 3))
 (segment (start 56.300001 84.240001) (end 57.150001 84.240001) (width 0.25) (layer F.Cu) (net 3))
 (segment (start 55.88 83.82) (end 56.300001 84.240001) (width 0.25) (layer F.Cu) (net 3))
 (segment (start 45.72 83.82) (end 55.88 83.82) (width 0.25) (layer F.Cu) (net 3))
 (segment (start 72.464999 70.649999) (end 72.860001 70.649999) (width 0.25) (layer F.Cu) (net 3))
 (segment (start 69.994999 73.119999) (end 72.464999 70.649999) (width 0.25) (layer F.Cu) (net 3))
 (segment (start 61.009002 83.82) (end 69.994999 74.834003) (width 0.25) (layer F.Cu) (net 3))
 (segment (start 60.070998 83.82) (end 61.009002 83.82) (width 0.25) (layer F.Cu) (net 3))
 (segment (start 69.994999 74.834003) (end 69.994999 73.119999) (width 0.25) (layer F.Cu) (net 3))
 (segment (start 59.650997 84.240001) (end 60.070998 83.82) (width 0.25) (layer F.Cu) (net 3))
 (segment (start 72.860001 70.649999) (end 73.66 69.85) (width 0.25) (layer F.Cu) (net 3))
 (segment (start 58.849999 84.240001) (end 59.650997 84.240001) (width 0.25) (layer F.Cu) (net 3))
 (segment (start 58 85.09) (end 58.849999 84.240001) (width 0.25) (layer F.Cu) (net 3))
 (segment (start 59.690001 83.399999) (end 60.54 82.55) (width 0.25) (layer F.Cu) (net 1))
 (segment (start 57.055001 83.725001) (end 59.364999 83.725001) (width 0.25) (layer F.Cu) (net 1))
 (segment (start 59.364999 83.725001) (end 59.690001 83.399999) (width 0.25) (layer F.Cu) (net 1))
 (segment (start 55.88 82.55) (end 57.055001 83.725001) (width 0.25) (layer F.Cu) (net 1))
 (segment (start 44.45 82.55) (end 55.88 82.55) (width 0.25) (layer F.Cu) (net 1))
 (segment (start 43.18 83.82) (end 44.45 82.55) (width 0.25) (layer F.Cu) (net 1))
 (segment (start 69.544989 73.545011) (end 69.544989 69.760009) (width 0.25) (layer F.Cu) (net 1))
 (segment (start 60.54 82.55) (end 69.544989 73.545011) (width 0.25) (layer F.Cu) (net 1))
 (segment (start 72.860001 66.839999) (end 73.66 66.04) (width 0.25) (layer F.Cu) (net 1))
 (segment (start 72.464999 66.839999) (end 72.860001 66.839999) (width 0.25) (layer F.Cu) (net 1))
 (segment (start 69.544989 69.760009) (end 72.464999 66.839999) (width 0.25) (layer F.Cu) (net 1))
 (segment (start 45.72 81.28) (end 55.87718 81.28) (width 0.25) (layer F.Cu) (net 19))
 (segment (start 56.797919 82.55) (end 58 82.55) (width 0.25) (layer F.Cu) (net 19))
 (segment (start 55.87718 81.629261) (end 56.797919 82.55) (width 0.25) (layer F.Cu) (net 19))
 (segment (start 55.87718 81.28) (end 55.87718 81.629261) (width 0.25) (layer F.Cu) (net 19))
 (segment (start 43.18 81.28) (end 44.45 80.01) (width 0.25) (layer F.Cu) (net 20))
 (segment (start 55.24359 80.01) (end 56.51359 81.28) (width 0.25) (layer F.Cu) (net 20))
 (segment (start 44.45 80.01) (end 55.24359 80.01) (width 0.25) (layer F.Cu) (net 20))
 (segment (start 59.27 81.28) (end 60.54 80.01) (width 0.25) (layer F.Cu) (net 20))
 (segment (start 56.51359 81.28) (end 59.27 81.28) (width 0.25) (layer F.Cu) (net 20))
 (segment (start 59.690001 61.380001) (end 60.54 62.23) (width 0.25) (layer F.Cu) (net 34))
 (segment (start 59.364999 61.054999) (end 59.690001 61.380001) (width 0.25) (layer F.Cu) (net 34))
 (segment (start 55.809997 62.135001) (end 56.889999 61.054999) (width 0.25) (layer F.Cu) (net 34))
 (segment (start 56.889999 61.054999) (end 59.364999 61.054999) (width 0.25) (layer F.Cu) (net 34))
 (segment (start 44.544999 62.135001) (end 55.809997 62.135001) (width 0.25) (layer F.Cu) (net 34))
 (segment (start 43.18 63.5) (end 44.544999 62.135001) (width 0.25) (layer F.Cu) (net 34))
 (segment (start 43.18 60.96) (end 45.72 60.96) (width 0.25) (layer B.Cu) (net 2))
 (segment (start 66.04 60.96) (end 71.12 66.04) (width 0.25) (layer B.Cu) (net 2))
 (segment (start 45.72 60.96) (end 66.04 60.96) (width 0.25) (layer B.Cu) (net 2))
 (segment (start 71.12 66.04) (end 71.12 69.85) (width 0.25) (layer B.Cu) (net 2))
 (segment (start 71.12 69.85) (end 71.12 73.66) (width 0.25) (layer B.Cu) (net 2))
 (segment (start 71.12 73.66) (end 71.12 77.47) (width 0.25) (layer B.Cu) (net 2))
 (segment (start 71.12 77.47) (end 71.12 81.28) (width 0.25) (layer B.Cu) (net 2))
 (segment (start 71.12 81.28) (end 71.12 85.09) (width 0.25) (layer B.Cu) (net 2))
 (segment (start 71.12 85.09) (end 71.12 88.9) (width 0.25) (layer B.Cu) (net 2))
 (segment (start 71.12 88.9) (end 71.12 92.71) (width 0.25) (layer B.Cu) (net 2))
 (segment (start 71.12 92.71) (end 71.12 96.52) (width 0.25) (layer B.Cu) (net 2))
 (segment (start 71.12 96.52) (end 71.12 100.33) (width 0.25) (layer B.Cu) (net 2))
 (segment (start 71.12 100.33) (end 71.12 104.14) (width 0.25) (layer B.Cu) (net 2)))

